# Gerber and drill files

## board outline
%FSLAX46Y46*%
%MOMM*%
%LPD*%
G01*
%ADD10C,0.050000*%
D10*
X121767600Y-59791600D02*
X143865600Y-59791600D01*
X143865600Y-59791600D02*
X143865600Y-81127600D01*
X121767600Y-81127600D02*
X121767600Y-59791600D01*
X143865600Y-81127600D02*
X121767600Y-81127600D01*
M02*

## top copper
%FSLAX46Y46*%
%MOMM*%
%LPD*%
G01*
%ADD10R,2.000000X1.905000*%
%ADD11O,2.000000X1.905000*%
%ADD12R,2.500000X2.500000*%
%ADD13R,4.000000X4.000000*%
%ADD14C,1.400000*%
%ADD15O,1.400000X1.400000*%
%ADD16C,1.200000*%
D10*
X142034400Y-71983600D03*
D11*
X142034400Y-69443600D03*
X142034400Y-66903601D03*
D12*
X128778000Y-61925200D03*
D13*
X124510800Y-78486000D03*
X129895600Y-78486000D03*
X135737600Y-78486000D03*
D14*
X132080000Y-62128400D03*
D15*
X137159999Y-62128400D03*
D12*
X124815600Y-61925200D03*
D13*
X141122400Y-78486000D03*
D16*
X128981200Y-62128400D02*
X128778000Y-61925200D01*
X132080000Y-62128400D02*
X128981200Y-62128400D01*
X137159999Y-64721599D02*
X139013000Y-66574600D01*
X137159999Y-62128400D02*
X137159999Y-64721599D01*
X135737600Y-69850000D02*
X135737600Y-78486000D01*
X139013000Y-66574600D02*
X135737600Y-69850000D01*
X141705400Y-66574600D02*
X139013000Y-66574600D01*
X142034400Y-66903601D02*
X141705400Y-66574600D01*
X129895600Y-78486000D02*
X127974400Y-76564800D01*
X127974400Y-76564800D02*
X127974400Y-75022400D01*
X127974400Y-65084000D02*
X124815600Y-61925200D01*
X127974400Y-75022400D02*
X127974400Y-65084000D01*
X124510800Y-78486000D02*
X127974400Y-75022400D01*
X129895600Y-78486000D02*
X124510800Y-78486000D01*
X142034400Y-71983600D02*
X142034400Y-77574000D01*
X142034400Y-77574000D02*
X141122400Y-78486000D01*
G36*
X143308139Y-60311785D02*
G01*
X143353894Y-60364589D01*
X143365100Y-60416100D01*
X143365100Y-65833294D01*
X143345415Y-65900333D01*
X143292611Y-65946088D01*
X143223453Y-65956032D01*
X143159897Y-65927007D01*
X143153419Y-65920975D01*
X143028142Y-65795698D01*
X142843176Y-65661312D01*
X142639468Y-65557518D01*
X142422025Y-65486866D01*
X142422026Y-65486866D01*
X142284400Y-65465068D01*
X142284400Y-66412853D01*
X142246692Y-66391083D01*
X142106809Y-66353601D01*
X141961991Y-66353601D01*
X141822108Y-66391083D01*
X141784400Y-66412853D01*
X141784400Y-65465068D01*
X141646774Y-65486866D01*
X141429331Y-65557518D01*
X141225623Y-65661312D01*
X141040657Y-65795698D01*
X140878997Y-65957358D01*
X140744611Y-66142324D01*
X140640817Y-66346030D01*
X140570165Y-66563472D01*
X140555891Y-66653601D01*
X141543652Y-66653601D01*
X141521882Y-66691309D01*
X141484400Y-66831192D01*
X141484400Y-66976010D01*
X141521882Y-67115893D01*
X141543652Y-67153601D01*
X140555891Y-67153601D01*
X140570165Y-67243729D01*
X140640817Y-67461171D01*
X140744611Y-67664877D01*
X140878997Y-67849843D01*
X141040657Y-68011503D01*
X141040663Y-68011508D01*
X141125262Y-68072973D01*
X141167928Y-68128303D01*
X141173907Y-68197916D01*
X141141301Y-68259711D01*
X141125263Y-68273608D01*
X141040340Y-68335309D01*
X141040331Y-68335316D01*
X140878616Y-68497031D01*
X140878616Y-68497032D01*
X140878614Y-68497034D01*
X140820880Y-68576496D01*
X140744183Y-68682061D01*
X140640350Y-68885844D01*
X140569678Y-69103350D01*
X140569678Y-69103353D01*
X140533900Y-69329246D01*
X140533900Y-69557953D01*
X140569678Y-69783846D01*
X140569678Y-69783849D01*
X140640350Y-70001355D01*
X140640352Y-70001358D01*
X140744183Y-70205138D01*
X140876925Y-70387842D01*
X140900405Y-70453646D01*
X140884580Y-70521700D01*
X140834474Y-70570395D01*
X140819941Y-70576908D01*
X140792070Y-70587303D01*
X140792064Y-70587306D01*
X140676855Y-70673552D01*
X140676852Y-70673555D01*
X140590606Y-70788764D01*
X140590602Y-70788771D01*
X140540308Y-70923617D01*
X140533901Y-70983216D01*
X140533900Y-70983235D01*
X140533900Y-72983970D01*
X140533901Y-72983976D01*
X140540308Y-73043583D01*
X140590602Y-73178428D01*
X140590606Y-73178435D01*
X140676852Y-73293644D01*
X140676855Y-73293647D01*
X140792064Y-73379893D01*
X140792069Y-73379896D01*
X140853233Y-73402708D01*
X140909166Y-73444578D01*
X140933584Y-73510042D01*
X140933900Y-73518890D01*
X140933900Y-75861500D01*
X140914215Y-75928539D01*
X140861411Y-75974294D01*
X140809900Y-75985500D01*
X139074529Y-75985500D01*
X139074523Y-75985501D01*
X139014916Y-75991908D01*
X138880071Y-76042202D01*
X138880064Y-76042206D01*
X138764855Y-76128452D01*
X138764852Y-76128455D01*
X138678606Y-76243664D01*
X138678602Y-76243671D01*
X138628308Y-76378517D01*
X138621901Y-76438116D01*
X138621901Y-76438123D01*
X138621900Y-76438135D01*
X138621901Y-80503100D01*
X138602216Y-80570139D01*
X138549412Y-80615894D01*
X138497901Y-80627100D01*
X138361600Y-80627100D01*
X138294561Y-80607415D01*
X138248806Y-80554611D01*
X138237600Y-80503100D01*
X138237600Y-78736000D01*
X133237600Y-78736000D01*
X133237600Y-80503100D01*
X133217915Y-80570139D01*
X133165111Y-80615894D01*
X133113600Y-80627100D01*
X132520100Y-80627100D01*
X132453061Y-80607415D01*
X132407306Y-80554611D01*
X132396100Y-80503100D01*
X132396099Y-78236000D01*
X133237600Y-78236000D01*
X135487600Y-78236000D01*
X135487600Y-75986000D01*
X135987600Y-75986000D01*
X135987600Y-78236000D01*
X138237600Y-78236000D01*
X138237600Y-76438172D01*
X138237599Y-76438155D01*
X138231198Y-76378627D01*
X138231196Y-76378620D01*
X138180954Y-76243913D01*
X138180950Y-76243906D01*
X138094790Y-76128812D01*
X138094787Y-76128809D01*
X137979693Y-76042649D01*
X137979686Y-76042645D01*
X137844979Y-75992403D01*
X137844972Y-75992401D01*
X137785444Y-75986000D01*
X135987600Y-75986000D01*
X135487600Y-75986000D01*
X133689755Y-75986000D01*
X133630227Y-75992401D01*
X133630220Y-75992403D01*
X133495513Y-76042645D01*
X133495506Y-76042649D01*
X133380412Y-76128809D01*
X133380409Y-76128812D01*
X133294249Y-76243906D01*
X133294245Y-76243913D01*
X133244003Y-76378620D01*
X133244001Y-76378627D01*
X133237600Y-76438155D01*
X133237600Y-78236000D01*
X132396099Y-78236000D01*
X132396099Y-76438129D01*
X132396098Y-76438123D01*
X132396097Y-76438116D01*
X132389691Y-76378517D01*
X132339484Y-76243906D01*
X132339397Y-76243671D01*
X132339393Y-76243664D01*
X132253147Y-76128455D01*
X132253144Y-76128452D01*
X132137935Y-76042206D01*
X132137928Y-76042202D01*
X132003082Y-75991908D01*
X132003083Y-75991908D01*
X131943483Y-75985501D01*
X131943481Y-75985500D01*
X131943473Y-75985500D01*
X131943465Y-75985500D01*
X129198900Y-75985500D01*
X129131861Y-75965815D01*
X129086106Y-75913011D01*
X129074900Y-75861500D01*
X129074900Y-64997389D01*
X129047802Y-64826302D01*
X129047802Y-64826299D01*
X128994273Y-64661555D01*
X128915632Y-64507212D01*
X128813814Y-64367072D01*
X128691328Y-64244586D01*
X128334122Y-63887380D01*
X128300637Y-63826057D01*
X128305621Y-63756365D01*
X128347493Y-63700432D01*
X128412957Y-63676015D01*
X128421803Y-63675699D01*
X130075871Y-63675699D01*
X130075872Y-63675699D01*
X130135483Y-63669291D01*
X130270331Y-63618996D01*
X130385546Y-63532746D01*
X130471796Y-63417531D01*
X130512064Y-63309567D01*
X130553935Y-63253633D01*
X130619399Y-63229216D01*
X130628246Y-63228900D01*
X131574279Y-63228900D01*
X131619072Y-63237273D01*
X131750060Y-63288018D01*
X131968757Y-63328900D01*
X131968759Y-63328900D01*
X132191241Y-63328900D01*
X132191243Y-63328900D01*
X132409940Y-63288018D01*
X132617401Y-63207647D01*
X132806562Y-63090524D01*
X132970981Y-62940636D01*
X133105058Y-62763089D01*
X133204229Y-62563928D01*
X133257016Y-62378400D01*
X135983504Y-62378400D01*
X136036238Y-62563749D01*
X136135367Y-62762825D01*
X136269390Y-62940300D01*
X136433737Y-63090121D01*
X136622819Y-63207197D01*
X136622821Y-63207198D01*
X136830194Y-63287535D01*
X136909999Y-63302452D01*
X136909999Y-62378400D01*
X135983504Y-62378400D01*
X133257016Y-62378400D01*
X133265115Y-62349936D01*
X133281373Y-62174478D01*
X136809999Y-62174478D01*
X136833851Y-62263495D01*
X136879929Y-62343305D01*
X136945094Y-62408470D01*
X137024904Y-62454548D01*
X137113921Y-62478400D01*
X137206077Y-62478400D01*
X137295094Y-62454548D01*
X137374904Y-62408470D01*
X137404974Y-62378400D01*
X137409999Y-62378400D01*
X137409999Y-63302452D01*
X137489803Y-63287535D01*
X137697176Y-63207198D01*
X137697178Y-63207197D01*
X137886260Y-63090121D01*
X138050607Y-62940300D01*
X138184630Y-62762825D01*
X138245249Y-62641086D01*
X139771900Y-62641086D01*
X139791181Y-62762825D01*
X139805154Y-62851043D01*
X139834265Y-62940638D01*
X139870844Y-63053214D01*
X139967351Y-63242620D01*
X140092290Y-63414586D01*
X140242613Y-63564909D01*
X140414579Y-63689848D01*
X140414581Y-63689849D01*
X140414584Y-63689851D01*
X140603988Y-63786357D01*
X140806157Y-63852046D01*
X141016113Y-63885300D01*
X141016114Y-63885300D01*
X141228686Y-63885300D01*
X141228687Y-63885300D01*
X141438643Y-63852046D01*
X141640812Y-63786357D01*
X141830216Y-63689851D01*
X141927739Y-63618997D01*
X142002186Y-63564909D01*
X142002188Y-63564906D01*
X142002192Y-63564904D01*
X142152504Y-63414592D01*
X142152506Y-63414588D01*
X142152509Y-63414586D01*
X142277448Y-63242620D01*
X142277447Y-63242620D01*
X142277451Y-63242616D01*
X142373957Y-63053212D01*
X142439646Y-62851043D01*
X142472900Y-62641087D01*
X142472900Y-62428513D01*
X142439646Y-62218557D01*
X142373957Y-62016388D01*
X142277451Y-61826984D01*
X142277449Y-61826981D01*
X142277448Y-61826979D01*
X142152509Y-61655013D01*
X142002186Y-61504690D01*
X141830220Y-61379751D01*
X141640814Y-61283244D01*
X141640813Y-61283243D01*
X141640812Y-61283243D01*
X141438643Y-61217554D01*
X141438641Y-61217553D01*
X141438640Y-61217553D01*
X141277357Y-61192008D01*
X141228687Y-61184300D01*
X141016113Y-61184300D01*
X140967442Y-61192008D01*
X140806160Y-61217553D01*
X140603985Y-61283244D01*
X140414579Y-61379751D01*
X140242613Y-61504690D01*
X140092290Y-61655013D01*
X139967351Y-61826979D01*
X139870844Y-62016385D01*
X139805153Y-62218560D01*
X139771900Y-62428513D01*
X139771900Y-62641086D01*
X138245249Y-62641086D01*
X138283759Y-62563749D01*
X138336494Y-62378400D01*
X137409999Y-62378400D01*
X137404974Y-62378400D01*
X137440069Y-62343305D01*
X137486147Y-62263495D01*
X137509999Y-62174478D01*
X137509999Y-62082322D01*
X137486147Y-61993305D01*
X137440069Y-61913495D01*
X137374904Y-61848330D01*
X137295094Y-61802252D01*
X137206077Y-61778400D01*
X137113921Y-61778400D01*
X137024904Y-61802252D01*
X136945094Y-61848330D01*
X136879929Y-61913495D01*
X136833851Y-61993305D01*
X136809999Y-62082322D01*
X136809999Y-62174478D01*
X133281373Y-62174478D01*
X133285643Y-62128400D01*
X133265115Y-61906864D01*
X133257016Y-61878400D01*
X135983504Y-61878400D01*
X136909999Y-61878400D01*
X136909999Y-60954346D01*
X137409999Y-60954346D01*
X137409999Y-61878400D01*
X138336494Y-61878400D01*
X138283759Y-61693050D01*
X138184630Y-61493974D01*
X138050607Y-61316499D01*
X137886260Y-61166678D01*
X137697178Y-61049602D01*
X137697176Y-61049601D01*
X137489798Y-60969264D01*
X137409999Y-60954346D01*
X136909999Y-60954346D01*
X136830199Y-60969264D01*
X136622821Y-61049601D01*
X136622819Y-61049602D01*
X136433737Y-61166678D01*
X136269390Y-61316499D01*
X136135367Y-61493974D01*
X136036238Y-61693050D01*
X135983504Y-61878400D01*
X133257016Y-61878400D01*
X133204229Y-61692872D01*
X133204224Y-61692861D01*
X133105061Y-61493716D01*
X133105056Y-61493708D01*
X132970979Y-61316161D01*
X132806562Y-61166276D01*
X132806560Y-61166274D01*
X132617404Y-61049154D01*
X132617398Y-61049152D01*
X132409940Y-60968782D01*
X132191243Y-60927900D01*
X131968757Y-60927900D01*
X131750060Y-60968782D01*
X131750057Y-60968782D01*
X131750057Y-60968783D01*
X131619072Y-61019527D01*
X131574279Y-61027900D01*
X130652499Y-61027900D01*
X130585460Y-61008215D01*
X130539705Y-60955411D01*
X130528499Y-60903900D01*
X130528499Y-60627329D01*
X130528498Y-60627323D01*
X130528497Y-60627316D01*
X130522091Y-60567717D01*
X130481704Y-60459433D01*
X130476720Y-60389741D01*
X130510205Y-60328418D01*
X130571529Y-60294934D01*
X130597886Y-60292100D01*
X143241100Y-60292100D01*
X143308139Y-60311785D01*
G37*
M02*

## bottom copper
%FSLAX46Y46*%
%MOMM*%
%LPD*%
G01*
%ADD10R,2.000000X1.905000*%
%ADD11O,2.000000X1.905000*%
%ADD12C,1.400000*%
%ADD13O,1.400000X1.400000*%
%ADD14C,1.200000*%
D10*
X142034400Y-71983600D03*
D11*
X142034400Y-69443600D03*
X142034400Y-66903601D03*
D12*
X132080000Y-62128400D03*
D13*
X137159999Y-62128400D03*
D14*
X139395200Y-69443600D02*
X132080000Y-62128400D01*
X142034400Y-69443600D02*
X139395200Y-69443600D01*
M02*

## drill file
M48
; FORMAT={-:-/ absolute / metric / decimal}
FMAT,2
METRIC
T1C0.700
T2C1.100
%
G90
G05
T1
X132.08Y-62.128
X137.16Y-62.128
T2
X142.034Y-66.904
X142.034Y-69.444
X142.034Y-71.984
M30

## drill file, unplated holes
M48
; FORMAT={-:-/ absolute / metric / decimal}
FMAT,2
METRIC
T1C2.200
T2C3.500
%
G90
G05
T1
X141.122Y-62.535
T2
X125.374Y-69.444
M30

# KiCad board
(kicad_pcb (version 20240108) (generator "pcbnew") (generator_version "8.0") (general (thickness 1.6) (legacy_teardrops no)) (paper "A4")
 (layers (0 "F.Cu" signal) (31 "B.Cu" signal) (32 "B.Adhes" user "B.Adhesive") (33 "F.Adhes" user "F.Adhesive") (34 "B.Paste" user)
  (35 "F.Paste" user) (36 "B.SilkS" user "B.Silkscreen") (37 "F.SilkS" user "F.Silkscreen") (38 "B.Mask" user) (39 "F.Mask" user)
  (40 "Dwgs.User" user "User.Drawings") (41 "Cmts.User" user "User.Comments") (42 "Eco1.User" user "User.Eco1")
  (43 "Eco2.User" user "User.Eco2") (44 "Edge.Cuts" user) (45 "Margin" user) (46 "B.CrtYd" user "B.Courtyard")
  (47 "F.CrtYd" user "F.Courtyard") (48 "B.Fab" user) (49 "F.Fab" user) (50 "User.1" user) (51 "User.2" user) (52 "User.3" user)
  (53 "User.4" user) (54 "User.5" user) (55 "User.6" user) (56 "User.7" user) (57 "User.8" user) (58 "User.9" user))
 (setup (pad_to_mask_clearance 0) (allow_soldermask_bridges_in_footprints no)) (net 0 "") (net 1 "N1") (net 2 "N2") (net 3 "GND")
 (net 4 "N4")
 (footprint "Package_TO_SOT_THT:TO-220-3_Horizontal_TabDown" (layer "F.Cu") (at 142.0344 71.9836 90)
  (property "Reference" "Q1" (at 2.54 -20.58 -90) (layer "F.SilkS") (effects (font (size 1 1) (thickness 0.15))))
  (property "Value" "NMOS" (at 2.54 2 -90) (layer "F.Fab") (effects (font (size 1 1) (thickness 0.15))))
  (pad "" np_thru_hole oval (at 2.54 -16.66 90) (size 3.5 3.5) (drill 3.5) (layers "*.Cu" "*.Mask"))
  (pad "1" thru_hole rect (at 0 0 90) (size 1.905 2) (drill 1.1) (layers "*.Cu" "*.Mask") (remove_unused_layers no) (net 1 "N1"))
  (pad "2" thru_hole oval (at 2.54 0 90) (size 1.905 2) (drill 1.1) (layers "*.Cu" "*.Mask") (remove_unused_layers no) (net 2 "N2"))
  (pad "3" thru_hole oval (at 5.079999 0 90) (size 1.905 2) (drill 1.1) (layers "*.Cu" "*.Mask") (remove_unused_layers no) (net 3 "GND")))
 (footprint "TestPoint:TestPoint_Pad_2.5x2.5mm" (layer "F.Cu") (at 128.778 61.9252)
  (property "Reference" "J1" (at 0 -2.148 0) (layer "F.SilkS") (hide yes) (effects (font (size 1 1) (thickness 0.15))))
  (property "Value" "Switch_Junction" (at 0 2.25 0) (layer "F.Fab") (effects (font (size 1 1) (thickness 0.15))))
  (pad "1" smd rect (at 0 0) (size 2.5 2.5) (layers "F.Cu" "F.Mask") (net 2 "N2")))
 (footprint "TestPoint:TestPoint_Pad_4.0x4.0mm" (layer "F.Cu") (at 124.5108 78.486)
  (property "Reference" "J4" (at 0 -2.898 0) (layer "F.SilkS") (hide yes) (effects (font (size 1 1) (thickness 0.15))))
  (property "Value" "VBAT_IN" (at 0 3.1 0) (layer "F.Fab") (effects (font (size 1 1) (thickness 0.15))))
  (pad "1" smd rect (at 0 0) (size 4 4) (layers "F.Cu" "F.Mask") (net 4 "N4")))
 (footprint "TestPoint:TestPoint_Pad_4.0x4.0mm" (layer "F.Cu") (at 129.8956 78.486)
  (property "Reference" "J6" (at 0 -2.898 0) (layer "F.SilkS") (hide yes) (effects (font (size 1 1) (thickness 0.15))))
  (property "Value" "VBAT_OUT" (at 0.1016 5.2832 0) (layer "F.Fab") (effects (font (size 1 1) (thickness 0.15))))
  (pad "1" smd rect (at 0 0) (size 4 4) (layers "F.Cu" "F.Mask") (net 4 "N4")))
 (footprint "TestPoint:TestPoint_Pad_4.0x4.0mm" (layer "F.Cu") (at 135.7376 78.486)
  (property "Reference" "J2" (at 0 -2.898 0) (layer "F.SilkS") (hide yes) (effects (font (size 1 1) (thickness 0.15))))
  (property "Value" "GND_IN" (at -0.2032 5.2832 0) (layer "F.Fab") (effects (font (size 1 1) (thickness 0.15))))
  (pad "1" smd rect (at 0 0) (size 4 4) (layers "F.Cu" "F.Mask") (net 3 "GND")))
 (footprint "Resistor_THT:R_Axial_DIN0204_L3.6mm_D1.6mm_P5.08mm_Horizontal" (layer "F.Cu") (at 132.08 62.1284)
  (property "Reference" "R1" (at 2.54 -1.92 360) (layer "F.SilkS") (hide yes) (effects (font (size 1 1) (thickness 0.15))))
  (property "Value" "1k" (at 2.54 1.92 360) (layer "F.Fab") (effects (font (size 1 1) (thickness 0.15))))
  (pad "1" thru_hole circle (at 0 0) (size 1.4 1.4) (drill 0.7) (layers "*.Cu" "*.Mask") (remove_unused_layers no) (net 2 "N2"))
  (pad "2" thru_hole oval (at 5.079999 0) (size 1.4 1.4) (drill 0.7) (layers "*.Cu" "*.Mask") (remove_unused_layers no) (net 3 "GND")))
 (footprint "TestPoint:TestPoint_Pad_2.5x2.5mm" (layer "F.Cu") (at 124.8156 61.9252)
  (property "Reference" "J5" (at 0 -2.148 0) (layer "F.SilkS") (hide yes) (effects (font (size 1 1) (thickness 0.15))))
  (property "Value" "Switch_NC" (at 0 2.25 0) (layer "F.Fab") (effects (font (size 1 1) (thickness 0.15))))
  (pad "1" smd rect (at 0 0) (size 2.5 2.5) (layers "F.Cu" "F.Mask") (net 4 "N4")))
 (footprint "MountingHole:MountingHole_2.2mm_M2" (layer "F.Cu") (at 141.1224 62.5348)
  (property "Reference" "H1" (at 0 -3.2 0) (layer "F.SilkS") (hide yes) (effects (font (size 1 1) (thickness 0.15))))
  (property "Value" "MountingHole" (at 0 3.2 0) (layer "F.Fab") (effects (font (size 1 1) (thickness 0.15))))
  (pad "" np_thru_hole circle (at 0 0) (size 2.2 2.2) (drill 2.2) (layers "*.Cu" "*.Mask")))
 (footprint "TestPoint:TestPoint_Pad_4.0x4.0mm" (layer "F.Cu") (at 141.1224 78.486)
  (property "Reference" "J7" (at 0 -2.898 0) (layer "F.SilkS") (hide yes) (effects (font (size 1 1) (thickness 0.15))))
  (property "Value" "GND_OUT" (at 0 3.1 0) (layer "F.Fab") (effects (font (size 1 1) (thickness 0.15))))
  (pad "1" smd rect (at 0 0) (size 4 4) (layers "F.Cu" "F.Mask") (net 1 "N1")))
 (gr_line (start 121.7676 59.7916) (end 143.8656 59.7916) (stroke (width 0.05) (type default)) (layer "Edge.Cuts"))
 (gr_line (start 143.8656 59.7916) (end 143.8656 81.1276) (stroke (width 0.05) (type default)) (layer "Edge.Cuts"))
 (gr_line (start 121.7676 81.1276) (end 121.7676 59.7916) (stroke (width 0.05) (type default)) (layer "Edge.Cuts"))
 (gr_line (start 143.8656 81.1276) (end 121.7676 81.1276) (stroke (width 0.05) (type default)) (layer "Edge.Cuts"))
 (segment (start 128.9812 62.1284) (end 128.778 61.9252) (width 1.2) (layer "F.Cu") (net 2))
 (segment (start 132.08 62.1284) (end 128.9812 62.1284) (width 1.2) (layer "F.Cu") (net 2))
 (segment (start 142.0344 69.4436) (end 139.3952 69.4436) (width 1.2) (layer "B.Cu") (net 2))
 (segment (start 139.3952 69.4436) (end 132.08 62.1284) (width 1.2) (layer "B.Cu") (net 2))
 (segment (start 141.7054 66.5746) (end 139.013 66.5746) (width 1.2) (layer "F.Cu") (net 3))
 (segment (start 137.159999 62.1284) (end 137.159999 64.721599) (width 1.2) (layer "F.Cu") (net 3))
 (segment (start 137.159999 64.721599) (end 139.013 66.5746) (width 1.2) (layer "F.Cu") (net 3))
 (segment (start 142.0344 66.903601) (end 141.7054 66.5746) (width 1.2) (layer "F.Cu") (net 3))
 (segment (start 135.7376 69.85) (end 135.7376 78.486) (width 1.2) (layer "F.Cu") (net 3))
 (segment (start 139.013 66.5746) (end 135.7376 69.85) (width 1.2) (layer "F.Cu") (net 3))
 (segment (start 127.9744 76.5648) (end 127.9744 75.0224) (width 1.2) (layer "F.Cu") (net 4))
 (segment (start 127.9744 65.084) (end 124.8156 61.9252) (width 1.2) (layer "F.Cu") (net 4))
 (segment (start 127.9744 75.0224) (end 127.9744 65.084) (width 1.2) (layer "F.Cu") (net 4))
 (segment (start 129.8956 78.486) (end 124.5108 78.486) (width 1.2) (layer "F.Cu") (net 4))
 (segment (start 124.5108 78.486) (end 127.9744 75.0224) (width 1.2) (layer "F.Cu") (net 4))
 (segment (start 129.8956 78.486) (end 127.9744 76.5648) (width 1.2) (layer "F.Cu") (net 4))
 (segment (start 142.0344 77.574) (end 141.1224 78.486) (width 1.2) (layer "F.Cu") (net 1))
 (segment (start 142.0344 71.9836) (end 142.0344 77.574) (width 1.2) (layer "F.Cu") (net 1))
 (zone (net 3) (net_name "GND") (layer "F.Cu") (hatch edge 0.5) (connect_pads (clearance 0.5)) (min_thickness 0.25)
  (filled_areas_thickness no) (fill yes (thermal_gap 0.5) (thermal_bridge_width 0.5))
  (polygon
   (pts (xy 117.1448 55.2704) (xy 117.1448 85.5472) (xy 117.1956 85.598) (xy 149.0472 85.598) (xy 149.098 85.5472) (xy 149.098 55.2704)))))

